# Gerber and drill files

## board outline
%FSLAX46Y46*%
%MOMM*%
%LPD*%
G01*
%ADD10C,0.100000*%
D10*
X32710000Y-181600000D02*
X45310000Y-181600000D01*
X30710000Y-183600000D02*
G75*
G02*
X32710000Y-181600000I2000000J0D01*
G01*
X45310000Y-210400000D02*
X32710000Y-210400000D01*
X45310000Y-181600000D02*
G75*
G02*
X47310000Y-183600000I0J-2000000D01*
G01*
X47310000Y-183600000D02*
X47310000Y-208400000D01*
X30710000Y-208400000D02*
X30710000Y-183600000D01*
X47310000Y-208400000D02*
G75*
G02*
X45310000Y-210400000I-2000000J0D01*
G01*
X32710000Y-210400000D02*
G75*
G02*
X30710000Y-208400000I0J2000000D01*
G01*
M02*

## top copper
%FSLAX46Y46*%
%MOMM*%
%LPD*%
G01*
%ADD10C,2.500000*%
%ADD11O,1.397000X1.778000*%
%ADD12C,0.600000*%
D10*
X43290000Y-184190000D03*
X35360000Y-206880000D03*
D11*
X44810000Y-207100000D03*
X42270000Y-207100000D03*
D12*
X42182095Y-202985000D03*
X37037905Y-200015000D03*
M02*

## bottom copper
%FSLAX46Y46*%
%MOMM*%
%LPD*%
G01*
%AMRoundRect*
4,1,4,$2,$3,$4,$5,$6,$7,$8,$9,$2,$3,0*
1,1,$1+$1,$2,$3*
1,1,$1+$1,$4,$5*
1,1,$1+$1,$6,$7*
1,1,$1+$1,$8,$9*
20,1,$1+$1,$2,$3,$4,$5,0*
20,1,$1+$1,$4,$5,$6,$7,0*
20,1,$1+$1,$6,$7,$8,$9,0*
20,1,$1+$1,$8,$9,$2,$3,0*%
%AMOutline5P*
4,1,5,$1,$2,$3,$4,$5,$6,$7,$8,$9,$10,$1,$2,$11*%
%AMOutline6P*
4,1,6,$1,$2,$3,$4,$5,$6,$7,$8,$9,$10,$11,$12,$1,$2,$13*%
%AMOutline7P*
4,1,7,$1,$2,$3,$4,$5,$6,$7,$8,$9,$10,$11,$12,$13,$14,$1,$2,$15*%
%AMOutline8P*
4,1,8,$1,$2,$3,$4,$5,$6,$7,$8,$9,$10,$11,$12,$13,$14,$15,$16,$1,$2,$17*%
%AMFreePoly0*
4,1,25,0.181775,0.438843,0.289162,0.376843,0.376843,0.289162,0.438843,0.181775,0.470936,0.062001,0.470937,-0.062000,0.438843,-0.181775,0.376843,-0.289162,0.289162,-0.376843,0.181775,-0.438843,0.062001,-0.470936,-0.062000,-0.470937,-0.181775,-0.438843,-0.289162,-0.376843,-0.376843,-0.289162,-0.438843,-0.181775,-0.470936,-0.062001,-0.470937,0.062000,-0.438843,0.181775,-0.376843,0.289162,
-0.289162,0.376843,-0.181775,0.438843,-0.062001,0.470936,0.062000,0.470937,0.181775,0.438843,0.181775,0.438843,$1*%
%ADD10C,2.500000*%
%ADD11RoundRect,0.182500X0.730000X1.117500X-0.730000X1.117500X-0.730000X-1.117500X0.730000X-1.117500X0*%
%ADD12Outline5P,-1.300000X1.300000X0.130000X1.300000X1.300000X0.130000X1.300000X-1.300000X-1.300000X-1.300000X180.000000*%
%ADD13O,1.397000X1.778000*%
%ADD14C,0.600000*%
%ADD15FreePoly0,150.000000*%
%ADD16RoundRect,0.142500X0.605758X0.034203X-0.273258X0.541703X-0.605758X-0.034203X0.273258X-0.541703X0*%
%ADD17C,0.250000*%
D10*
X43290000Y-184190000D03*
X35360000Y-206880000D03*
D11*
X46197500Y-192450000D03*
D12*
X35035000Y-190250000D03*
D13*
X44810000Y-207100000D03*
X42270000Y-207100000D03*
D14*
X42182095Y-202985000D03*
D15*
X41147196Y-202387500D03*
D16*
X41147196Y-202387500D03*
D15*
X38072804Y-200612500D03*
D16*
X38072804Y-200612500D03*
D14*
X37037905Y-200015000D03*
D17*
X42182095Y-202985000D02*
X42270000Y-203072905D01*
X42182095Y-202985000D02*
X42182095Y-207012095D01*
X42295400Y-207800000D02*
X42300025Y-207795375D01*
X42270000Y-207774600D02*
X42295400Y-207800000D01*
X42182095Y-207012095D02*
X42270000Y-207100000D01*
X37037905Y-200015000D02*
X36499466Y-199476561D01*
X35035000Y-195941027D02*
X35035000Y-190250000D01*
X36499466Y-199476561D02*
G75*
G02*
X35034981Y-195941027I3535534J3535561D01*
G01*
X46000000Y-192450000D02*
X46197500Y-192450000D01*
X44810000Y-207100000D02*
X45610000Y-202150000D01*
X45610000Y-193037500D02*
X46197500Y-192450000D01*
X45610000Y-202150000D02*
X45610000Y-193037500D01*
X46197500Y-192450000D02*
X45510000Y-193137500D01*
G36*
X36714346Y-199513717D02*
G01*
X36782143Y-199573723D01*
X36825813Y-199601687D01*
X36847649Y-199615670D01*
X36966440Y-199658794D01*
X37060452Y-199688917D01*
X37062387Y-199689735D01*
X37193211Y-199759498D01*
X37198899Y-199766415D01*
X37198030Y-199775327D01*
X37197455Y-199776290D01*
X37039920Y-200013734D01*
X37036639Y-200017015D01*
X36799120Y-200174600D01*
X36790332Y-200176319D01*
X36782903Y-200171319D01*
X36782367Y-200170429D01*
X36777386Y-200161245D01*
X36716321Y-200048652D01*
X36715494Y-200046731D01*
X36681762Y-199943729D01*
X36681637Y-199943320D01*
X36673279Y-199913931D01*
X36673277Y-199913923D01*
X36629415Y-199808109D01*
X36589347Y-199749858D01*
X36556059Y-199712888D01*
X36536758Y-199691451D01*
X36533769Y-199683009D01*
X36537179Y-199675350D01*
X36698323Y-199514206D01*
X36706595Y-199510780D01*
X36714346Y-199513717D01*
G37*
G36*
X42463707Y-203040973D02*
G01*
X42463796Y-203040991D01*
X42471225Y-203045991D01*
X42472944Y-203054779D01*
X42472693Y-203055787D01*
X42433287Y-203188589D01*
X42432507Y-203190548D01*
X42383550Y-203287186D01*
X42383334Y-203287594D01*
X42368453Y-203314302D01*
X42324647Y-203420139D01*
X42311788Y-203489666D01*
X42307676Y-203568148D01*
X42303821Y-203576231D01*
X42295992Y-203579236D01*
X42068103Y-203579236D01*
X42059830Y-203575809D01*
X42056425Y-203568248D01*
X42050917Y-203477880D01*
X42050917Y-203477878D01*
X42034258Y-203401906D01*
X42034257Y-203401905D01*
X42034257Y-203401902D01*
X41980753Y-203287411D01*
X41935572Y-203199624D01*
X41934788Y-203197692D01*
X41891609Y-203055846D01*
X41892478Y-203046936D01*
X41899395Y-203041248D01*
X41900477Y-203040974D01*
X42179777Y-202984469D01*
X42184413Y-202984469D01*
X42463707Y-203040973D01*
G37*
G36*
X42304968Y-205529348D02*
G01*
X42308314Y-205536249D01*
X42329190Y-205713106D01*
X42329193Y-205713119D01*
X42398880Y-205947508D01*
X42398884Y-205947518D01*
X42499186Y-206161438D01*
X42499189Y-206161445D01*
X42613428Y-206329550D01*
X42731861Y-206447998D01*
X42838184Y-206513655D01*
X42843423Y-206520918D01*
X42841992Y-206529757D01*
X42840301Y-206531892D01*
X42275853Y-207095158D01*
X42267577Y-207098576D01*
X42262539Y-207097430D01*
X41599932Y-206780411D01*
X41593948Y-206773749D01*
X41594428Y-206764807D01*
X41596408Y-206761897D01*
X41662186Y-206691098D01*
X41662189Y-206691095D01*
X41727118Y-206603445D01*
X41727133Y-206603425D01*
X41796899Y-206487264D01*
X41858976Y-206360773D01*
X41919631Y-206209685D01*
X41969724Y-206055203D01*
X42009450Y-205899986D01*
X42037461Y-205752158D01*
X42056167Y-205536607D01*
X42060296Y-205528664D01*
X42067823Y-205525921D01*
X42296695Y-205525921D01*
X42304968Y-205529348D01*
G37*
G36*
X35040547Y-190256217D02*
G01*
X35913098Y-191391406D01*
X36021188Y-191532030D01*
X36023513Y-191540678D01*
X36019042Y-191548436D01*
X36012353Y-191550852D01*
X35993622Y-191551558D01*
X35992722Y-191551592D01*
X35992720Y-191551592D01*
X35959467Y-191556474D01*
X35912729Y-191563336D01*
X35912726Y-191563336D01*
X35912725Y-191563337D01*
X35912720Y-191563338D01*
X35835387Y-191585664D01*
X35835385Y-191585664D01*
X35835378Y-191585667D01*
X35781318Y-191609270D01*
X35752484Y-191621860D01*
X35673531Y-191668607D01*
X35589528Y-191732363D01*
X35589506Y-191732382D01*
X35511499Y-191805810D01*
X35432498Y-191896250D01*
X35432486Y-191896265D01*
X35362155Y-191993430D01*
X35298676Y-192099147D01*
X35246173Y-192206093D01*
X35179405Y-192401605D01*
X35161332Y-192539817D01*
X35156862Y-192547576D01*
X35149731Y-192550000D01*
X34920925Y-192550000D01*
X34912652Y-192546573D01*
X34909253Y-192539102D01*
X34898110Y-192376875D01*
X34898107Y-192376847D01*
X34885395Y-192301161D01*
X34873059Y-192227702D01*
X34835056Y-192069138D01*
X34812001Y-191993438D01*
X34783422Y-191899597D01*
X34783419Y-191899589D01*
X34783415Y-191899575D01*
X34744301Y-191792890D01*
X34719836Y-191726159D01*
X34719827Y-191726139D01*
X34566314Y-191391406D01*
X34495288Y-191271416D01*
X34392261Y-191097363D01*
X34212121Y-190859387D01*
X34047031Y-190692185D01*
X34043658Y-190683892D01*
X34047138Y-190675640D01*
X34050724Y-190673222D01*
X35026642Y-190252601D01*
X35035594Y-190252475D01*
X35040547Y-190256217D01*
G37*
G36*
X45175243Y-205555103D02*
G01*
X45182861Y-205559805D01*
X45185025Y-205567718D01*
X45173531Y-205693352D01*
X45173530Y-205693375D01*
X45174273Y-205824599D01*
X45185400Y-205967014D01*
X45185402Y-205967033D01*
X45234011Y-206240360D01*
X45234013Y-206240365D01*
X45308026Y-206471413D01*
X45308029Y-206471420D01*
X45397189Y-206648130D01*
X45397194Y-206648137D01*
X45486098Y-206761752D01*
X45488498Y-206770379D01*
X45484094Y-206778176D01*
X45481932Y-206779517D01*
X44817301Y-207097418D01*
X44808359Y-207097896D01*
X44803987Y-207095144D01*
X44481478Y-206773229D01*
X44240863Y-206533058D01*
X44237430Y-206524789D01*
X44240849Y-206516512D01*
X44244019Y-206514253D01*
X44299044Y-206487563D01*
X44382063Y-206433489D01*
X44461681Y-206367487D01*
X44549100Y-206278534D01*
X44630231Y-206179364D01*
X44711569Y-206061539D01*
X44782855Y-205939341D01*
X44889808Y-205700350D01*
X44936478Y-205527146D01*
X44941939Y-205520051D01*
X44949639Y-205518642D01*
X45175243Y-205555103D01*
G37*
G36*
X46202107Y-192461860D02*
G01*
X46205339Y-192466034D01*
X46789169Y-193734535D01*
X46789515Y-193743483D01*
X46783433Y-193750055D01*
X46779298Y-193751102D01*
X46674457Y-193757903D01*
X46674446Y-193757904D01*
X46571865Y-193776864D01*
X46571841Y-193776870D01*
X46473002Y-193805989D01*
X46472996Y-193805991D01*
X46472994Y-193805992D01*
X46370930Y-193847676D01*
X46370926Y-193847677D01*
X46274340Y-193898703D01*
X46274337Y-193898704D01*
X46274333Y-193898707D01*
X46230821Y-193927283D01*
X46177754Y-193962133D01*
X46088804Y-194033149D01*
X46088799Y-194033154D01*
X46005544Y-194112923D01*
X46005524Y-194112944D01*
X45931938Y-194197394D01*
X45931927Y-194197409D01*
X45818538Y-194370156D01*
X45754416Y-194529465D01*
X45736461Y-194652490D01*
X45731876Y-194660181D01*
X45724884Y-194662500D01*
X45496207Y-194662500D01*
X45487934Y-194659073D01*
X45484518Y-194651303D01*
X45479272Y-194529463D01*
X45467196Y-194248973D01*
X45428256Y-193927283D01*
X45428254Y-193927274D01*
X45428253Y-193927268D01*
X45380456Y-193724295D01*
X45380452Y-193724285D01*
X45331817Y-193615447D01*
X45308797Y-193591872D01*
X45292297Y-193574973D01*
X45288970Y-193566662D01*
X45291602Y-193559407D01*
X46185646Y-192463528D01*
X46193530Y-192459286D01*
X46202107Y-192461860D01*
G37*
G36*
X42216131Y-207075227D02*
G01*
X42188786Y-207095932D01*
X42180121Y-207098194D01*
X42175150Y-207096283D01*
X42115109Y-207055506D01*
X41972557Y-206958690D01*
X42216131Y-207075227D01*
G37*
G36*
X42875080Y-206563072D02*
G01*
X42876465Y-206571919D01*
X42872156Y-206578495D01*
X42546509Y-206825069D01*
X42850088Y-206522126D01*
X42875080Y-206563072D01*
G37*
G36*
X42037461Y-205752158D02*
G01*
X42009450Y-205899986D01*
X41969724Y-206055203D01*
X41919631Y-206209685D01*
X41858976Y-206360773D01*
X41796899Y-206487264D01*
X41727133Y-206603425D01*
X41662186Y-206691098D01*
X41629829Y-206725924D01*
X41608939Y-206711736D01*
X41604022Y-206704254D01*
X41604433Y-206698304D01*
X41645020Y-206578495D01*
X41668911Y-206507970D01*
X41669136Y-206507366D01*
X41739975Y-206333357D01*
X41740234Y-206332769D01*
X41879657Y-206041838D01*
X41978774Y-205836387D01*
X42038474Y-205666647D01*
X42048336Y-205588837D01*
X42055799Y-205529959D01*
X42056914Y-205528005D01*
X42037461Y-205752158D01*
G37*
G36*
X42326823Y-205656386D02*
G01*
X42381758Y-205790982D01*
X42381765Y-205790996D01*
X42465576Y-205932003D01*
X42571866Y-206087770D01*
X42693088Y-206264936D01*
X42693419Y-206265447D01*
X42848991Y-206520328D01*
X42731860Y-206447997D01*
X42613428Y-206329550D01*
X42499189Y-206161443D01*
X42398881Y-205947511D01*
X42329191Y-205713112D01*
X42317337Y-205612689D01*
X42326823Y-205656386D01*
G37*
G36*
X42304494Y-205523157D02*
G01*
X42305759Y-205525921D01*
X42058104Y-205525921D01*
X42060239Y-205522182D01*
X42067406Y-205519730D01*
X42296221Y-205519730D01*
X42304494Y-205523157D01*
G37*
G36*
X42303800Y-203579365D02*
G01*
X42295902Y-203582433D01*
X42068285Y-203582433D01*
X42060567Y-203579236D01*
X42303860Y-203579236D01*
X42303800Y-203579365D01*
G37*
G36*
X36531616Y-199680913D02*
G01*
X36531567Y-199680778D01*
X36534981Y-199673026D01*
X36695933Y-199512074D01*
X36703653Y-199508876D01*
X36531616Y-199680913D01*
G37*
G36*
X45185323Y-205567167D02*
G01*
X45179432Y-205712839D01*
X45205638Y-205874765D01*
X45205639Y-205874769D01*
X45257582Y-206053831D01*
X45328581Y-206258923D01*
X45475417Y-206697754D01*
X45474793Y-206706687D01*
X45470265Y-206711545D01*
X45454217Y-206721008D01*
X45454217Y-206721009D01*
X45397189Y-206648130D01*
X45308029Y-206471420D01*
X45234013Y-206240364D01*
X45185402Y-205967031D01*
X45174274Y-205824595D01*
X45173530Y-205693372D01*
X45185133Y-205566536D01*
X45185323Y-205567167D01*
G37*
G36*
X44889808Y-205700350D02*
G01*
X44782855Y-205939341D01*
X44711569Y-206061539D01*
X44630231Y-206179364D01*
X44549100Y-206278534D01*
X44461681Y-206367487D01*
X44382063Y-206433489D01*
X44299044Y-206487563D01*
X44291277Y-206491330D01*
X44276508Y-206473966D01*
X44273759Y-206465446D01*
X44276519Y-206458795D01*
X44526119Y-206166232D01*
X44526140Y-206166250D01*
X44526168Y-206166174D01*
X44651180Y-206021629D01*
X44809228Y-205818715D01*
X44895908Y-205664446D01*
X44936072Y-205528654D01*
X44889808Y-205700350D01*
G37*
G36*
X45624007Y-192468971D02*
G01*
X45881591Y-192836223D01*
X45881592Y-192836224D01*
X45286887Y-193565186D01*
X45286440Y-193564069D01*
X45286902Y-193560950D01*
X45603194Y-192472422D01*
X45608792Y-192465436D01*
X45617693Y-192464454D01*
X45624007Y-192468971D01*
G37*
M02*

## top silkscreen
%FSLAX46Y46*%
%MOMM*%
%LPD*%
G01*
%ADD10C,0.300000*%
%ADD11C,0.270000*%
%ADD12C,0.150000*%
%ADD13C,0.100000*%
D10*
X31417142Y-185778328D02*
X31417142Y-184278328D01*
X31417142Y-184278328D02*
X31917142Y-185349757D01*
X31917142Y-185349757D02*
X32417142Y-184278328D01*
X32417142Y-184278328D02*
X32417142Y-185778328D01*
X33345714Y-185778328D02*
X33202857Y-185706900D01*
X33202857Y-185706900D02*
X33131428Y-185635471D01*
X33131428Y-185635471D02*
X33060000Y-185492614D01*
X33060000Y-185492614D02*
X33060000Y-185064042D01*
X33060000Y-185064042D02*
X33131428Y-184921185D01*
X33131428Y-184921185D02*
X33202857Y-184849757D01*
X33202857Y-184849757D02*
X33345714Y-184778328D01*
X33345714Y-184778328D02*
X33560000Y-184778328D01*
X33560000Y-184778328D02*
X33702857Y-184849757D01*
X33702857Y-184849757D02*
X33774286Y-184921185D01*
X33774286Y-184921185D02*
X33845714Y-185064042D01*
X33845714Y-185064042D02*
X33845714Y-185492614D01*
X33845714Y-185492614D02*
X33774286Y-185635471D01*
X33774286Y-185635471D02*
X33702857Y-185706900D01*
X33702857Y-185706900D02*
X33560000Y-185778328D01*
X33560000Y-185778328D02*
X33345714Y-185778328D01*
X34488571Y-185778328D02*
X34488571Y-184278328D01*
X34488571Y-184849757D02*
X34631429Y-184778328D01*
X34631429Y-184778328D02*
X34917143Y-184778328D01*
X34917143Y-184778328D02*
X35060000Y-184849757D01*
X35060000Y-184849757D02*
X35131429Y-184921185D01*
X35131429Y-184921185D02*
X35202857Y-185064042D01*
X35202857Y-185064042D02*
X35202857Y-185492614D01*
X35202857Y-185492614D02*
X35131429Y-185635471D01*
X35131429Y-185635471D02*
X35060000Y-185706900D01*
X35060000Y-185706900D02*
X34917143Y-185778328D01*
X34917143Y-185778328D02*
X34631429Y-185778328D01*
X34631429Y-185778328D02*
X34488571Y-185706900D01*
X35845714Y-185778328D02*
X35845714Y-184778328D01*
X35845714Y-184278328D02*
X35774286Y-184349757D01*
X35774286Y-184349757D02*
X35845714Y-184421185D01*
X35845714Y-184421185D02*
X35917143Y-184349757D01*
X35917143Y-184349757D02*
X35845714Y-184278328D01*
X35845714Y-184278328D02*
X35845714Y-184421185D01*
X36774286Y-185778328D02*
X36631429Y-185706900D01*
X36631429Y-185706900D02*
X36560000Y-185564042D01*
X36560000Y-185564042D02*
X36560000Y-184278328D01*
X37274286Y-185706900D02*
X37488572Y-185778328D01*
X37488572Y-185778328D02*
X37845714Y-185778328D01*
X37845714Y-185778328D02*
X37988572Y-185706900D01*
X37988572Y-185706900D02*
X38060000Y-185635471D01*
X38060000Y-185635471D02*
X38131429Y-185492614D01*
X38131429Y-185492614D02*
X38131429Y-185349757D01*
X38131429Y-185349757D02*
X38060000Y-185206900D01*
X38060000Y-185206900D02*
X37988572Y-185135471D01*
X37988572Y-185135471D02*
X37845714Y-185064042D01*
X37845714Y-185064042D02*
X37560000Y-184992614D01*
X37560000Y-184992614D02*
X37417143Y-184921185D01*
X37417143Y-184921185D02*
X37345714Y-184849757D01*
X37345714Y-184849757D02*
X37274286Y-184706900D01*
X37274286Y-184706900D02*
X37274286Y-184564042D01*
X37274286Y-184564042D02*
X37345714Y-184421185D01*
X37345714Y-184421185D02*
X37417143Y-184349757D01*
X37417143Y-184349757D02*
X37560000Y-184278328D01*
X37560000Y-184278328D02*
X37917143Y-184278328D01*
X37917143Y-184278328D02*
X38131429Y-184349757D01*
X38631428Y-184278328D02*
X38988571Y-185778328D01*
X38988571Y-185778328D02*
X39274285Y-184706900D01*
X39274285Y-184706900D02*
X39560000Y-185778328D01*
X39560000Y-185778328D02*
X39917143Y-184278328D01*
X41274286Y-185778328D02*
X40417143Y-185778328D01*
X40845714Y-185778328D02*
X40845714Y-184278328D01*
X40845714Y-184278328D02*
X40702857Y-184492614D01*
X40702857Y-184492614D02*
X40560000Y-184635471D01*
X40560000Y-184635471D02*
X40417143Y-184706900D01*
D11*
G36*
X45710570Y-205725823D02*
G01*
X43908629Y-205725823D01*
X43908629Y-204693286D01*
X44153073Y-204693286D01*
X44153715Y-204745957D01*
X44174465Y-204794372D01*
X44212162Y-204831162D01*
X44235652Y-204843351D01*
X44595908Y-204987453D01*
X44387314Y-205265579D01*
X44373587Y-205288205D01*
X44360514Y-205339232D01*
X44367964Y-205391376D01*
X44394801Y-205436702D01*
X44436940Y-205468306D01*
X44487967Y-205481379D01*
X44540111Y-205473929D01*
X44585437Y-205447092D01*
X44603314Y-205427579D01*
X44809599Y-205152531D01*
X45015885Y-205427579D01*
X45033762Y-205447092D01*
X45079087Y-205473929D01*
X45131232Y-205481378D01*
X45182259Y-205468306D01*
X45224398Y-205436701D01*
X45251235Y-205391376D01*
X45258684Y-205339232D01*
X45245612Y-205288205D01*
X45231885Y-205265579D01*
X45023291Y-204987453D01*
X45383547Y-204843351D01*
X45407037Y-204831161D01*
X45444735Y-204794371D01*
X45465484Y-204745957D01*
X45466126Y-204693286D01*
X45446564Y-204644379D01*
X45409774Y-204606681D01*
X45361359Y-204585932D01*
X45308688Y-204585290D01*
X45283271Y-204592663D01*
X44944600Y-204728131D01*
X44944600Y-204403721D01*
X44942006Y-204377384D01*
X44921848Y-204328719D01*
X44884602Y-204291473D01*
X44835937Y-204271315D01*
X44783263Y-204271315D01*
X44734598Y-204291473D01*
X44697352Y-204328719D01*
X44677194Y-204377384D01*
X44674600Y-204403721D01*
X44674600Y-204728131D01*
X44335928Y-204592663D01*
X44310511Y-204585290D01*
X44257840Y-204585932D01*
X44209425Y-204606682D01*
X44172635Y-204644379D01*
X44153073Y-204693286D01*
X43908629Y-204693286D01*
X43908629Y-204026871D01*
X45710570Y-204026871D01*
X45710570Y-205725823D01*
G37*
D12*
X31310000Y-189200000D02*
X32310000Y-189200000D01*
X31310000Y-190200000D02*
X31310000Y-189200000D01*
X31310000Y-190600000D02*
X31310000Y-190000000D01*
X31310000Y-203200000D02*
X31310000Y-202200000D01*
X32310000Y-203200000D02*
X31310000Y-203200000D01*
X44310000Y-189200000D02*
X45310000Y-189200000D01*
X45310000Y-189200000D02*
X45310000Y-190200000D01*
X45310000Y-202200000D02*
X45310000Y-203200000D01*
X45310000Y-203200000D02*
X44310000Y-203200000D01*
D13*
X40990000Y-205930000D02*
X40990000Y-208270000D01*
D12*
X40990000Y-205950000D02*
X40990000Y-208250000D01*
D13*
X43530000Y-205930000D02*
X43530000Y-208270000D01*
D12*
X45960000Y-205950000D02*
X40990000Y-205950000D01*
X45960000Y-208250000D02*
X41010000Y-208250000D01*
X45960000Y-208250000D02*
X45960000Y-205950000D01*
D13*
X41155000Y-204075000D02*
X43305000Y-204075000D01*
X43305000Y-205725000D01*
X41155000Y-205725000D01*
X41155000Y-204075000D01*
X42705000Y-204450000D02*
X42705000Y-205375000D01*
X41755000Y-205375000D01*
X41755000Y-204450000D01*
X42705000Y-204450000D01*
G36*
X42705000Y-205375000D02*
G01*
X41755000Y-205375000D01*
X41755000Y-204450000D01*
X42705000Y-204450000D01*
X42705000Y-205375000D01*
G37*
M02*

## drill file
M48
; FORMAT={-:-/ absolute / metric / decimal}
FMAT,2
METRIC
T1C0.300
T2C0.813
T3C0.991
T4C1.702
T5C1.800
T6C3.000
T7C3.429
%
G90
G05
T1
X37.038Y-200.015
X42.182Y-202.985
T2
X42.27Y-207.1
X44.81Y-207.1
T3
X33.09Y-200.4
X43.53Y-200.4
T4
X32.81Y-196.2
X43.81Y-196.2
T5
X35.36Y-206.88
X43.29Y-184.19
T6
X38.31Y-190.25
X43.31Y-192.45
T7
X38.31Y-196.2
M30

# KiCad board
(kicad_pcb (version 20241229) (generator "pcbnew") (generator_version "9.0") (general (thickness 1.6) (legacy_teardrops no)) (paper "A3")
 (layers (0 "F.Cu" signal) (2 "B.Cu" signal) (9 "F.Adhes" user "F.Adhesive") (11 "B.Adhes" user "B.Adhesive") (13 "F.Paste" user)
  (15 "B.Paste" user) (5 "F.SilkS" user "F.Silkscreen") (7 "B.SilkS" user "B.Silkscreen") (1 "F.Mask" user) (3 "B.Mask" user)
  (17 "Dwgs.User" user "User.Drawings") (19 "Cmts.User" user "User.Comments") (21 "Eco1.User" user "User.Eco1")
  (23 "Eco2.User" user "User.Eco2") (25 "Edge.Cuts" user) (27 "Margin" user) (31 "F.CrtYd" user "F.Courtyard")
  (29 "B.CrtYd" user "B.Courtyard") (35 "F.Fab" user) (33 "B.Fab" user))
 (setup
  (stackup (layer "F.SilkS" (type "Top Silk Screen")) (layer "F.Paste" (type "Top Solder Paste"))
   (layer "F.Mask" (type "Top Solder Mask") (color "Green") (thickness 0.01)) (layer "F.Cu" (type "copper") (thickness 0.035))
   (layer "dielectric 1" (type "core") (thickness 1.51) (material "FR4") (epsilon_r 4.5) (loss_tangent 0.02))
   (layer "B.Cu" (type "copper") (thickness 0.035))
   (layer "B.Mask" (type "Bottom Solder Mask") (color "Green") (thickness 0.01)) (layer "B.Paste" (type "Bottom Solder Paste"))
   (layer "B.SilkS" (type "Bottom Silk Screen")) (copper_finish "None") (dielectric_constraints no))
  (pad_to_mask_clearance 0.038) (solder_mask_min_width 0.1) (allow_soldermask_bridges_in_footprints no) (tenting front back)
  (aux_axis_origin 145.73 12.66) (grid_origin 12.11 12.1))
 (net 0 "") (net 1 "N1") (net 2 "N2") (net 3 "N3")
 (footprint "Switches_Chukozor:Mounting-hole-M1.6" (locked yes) (layer "F.Cu") (at 43.29 184.19)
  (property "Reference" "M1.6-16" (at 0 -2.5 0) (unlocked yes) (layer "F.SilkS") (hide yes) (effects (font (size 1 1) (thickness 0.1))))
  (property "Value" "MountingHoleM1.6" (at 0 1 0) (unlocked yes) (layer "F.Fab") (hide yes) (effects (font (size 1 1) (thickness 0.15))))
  (pad "" np_thru_hole circle (at 0 0) (size 2.5 2.5) (drill 1.8) (layers "*.Cu" "*.Mask") (clearance 0.2)))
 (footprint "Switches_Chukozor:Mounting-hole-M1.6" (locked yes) (layer "F.Cu") (at 35.36 206.88)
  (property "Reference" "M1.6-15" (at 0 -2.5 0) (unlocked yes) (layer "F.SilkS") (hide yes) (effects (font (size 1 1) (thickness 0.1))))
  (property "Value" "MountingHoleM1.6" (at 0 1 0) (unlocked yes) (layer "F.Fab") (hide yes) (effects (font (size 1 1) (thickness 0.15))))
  (pad "" np_thru_hole circle (at 0 0) (size 2.5 2.5) (drill 1.8) (layers "*.Cu" "*.Mask") (clearance 0.2)))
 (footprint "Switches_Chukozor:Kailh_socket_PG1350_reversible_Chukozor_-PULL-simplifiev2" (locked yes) (layer "F.Cu") (at 38.31 196.2 180)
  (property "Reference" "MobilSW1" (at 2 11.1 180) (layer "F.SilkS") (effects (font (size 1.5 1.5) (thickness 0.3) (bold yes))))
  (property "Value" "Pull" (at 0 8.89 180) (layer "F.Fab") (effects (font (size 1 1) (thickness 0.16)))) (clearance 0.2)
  (fp_line (start 7 7) (end 6 7) (stroke (width 0.15) (type solid)) (layer "F.SilkS"))
  (fp_line (start 7 6) (end 7 7) (stroke (width 0.15) (type solid)) (layer "F.SilkS"))
  (fp_line (start 7 5.6) (end 7 6.2) (stroke (width 0.15) (type solid)) (layer "F.SilkS"))
  (fp_line (start 7 -7) (end 7 -6) (stroke (width 0.15) (type solid)) (layer "F.SilkS"))
  (fp_line (start 6 -7) (end 7 -7) (stroke (width 0.15) (type solid)) (layer "F.SilkS"))
  (fp_line (start -6 7) (end -7 7) (stroke (width 0.15) (type solid)) (layer "F.SilkS"))
  (fp_line (start -7 7) (end -7 6) (stroke (width 0.15) (type solid)) (layer "F.SilkS"))
  (fp_line (start -7 -6) (end -7 -7) (stroke (width 0.15) (type solid)) (layer "F.SilkS"))
  (fp_line (start -7 -7) (end -6 -7) (stroke (width 0.15) (type solid)) (layer "F.SilkS"))
  (pad "" np_thru_hole circle (at -5.5 0 180) (size 1.7018 1.7018) (drill 1.7018) (layers "*.Cu" "*.Mask"))
  (pad "" np_thru_hole circle (at -5.22 -4.2 180) (size 0.9906 0.9906) (drill 0.9906) (layers "*.Cu" "*.Mask"))
  (pad "" np_thru_hole circle (at -5 3.75 180) (size 3 3) (drill 3) (layers "*.Cu" "*.Mask"))
  (pad "" np_thru_hole circle (at 0 0 180) (size 3.429 3.429) (drill 3.429) (layers "*.Cu" "*.Mask") (solder_mask_margin 0.1)
   (clearance 0.3))
  (pad "" np_thru_hole circle (at 0 5.95 180) (size 3 3) (drill 3) (layers "*.Cu" "*.Mask"))
  (pad "" np_thru_hole circle (at 5.22 -4.2 180) (size 0.9906 0.9906) (drill 0.9906) (layers "*.Cu" "*.Mask"))
  (pad "" np_thru_hole circle (at 5.5 0 180) (size 1.7018 1.7018) (drill 1.7018) (layers "*.Cu" "*.Mask"))
  (pad "1" smd roundrect (at -7.8875 3.75 180) (size 1.825 2.6) (layers "B.Cu" "B.Mask") (roundrect_rratio 0.1) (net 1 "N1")
   (teardrops (best_length_ratio 0.5) (max_length 1) (best_width_ratio 1) (max_width 2) (curved_edges yes) (filter_ratio 0.9) (enabled yes)
    (allow_two_segments yes) (prefer_zone_connections yes)))
  (pad "2" smd roundrect (at 3.275 5.95 180) (size 2.6 2.6) (layers "B.Cu" "B.Mask") (roundrect_rratio 0) (chamfer_ratio 0.45)
   (chamfer top_right) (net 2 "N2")
   (teardrops (best_length_ratio 0.5) (max_length 1) (best_width_ratio 1) (max_width 2) (curved_edges yes) (filter_ratio 0.9) (enabled yes)
    (allow_two_segments yes) (prefer_zone_connections yes))))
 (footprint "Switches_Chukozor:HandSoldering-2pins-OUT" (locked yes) (layer "F.Cu") (at 43.4146 207.1)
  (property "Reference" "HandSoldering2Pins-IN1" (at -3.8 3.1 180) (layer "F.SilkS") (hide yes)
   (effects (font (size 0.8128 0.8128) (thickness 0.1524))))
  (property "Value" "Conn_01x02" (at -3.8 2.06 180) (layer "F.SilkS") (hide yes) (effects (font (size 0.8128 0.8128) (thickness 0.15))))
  (fp_line (start -2.4246 -1.17) (end -2.4246 1.17) (stroke (width 0.1) (type default)) (layer "F.SilkS"))
  (fp_line (start -2.4246 -1.15) (end -2.4246 1.15) (stroke (width 0.15) (type solid)) (layer "F.SilkS"))
  (fp_line (start 0.1154 -1.17) (end 0.1154 1.17) (stroke (width 0.1) (type default)) (layer "F.SilkS"))
  (fp_line (start 2.5454 -1.15) (end -2.4246 -1.15) (stroke (width 0.15) (type solid)) (layer "F.SilkS"))
  (fp_line (start 2.5454 1.15) (end -2.4046 1.15) (stroke (width 0.15) (type solid)) (layer "F.SilkS"))
  (fp_line (start 2.5454 1.15) (end 2.5454 -1.15) (stroke (width 0.15) (type solid)) (layer "F.SilkS"))
  (fp_rect (start -0.1096 -3.025) (end -2.2596 -1.375) (stroke (width 0.1) (type default)) (fill no) (layer "F.SilkS"))
  (fp_poly
   (pts (xy -0.7096 -2.65) (xy -0.7096 -1.725) (xy -1.6596 -1.725) (xy -1.6596 -2.65)) (stroke (width 0.1) (type solid)) (fill yes)
   (layer "F.SilkS"))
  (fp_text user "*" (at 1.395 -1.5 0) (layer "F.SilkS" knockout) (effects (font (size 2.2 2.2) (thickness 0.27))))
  (pad "1" thru_hole oval (at 1.3954 0) (size 1.397 1.778) (drill 0.8128) (layers "*.Cu" "*.Mask") (remove_unused_layers no) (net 1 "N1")
   (teardrops (best_length_ratio 0.5) (max_length 1) (best_width_ratio 1) (max_width 2) (curved_edges yes) (filter_ratio 0.9) (enabled yes)
    (allow_two_segments yes) (prefer_zone_connections yes)))
  (pad "2" thru_hole oval (at -1.1446 0) (size 1.397 1.778) (drill 0.8128) (layers "*.Cu" "*.Mask") (remove_unused_layers no) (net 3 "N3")
   (teardrops (best_length_ratio 0.5) (max_length 1) (best_width_ratio 1) (max_width 2) (curved_edges yes) (filter_ratio 0.9) (enabled yes)
    (allow_two_segments yes) (prefer_zone_connections yes))))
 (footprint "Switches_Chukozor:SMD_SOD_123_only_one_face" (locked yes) (layer "F.Cu") (at 39.61 201.5 150)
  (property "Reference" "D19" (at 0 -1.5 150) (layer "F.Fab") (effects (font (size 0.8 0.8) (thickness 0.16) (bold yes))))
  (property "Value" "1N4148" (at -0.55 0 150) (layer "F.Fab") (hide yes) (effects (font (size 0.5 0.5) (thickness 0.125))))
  (pad "1" thru_hole circle (at -2.97 0 150) (size 0.6 0.6) (drill 0.3) (layers "*.Cu") (remove_unused_layers no) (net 3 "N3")
   (teardrops (best_length_ratio 0.5) (max_length 1) (best_width_ratio 1) (max_width 2) (curved_edges yes) (filter_ratio 0.9) (enabled yes)
    (allow_two_segments yes) (prefer_zone_connections yes)))
  (pad "1" smd custom (at -1.775001 0 150) (size 0.95 0.95) (layers "B.Cu") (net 3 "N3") (thermal_bridge_angle 90)
   (options (clearance outline) (anchor circle)) (primitives)
   (teardrops (best_length_ratio 0.5) (max_length 1) (best_width_ratio 1) (max_width 2) (curved_edges no) (filter_ratio 0.9) (enabled no)
    (allow_two_segments no) (prefer_zone_connections yes)))
  (pad "1" smd roundrect (at -1.775001 0 150) (size 1.3 0.95) (layers "B.Cu" "B.Mask") (roundrect_rratio 0.15) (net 3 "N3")
   (teardrops (best_length_ratio 0.5) (max_length 1) (best_width_ratio 1) (max_width 2) (curved_edges yes) (filter_ratio 0.9) (enabled yes)
    (allow_two_segments yes) (prefer_zone_connections yes)))
  (pad "2" smd custom (at 1.775001 0 150) (size 0.95 0.95) (layers "B.Cu") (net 2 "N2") (thermal_bridge_angle 90)
   (options (clearance outline) (anchor circle)) (primitives)
   (teardrops (best_length_ratio 0.5) (max_length 1) (best_width_ratio 1) (max_width 2) (curved_edges no) (filter_ratio 0.9) (enabled no)
    (allow_two_segments no) (prefer_zone_connections yes)))
  (pad "2" smd roundrect (at 1.775001 0 150) (size 1.3 0.95) (layers "B.Cu" "B.Mask") (roundrect_rratio 0.15) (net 2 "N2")
   (teardrops (best_length_ratio 0.5) (max_length 1) (best_width_ratio 1) (max_width 2) (curved_edges yes) (filter_ratio 0.9) (enabled yes)
    (allow_two_segments yes) (prefer_zone_connections yes)))
  (pad "2" thru_hole circle (at 2.97 0 150) (size 0.6 0.6) (drill 0.3) (layers "*.Cu") (remove_unused_layers no) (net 2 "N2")
   (teardrops (best_length_ratio 0.5) (max_length 1) (best_width_ratio 1) (max_width 2) (curved_edges yes) (filter_ratio 0.9) (enabled yes)
    (allow_two_segments yes) (prefer_zone_connections yes))))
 (gr_line (start 32.71 181.6) (end 45.31 181.6) (stroke (width 0.1) (type default)) (locked yes) (layer "Edge.Cuts"))
 (gr_arc (start 30.71 183.6) (mid 31.295786 182.185786) (end 32.71 181.6) (stroke (width 0.1) (type default)) (locked yes)
  (layer "Edge.Cuts"))
 (gr_line (start 45.31 210.4) (end 32.71 210.4) (stroke (width 0.1) (type default)) (locked yes) (layer "Edge.Cuts"))
 (gr_arc (start 45.31 181.6) (mid 46.724214 182.185786) (end 47.31 183.6) (stroke (width 0.1) (type default)) (locked yes)
  (layer "Edge.Cuts"))
 (gr_line (start 47.31 183.6) (end 47.31 208.4) (stroke (width 0.1) (type default)) (locked yes) (layer "Edge.Cuts"))
 (gr_line (start 30.71 208.4) (end 30.71 183.6) (stroke (width 0.1) (type default)) (locked yes) (layer "Edge.Cuts"))
 (gr_arc (start 47.31 208.4) (mid 46.724214 209.814214) (end 45.31 210.4) (stroke (width 0.1) (type default)) (locked yes)
  (layer "Edge.Cuts"))
 (gr_arc (start 32.71 210.4) (mid 31.295786 209.814214) (end 30.71 208.4) (stroke (width 0.1) (type default)) (locked yes)
  (layer "Edge.Cuts"))
 (segment (start 42.182095 202.985) (end 42.27 203.072905) (width 0.25) (layer "B.Cu") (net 3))
 (segment (start 42.182095 202.985) (end 42.182095 207.012095) (width 0.25) (layer "B.Cu") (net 3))
 (segment (start 42.2954 207.8) (end 42.300025 207.795375) (width 0.25) (layer "B.Cu") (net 3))
 (segment (start 42.27 207.7746) (end 42.2954 207.8) (width 0.25) (layer "B.Cu") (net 3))
 (segment (start 42.182095 207.012095) (end 42.27 207.1) (width 0.25) (layer "B.Cu") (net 3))
 (segment (start 37.037905 200.015) (end 36.499466 199.476561) (width 0.25) (layer "B.Cu") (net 2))
 (segment (start 35.035 195.941027) (end 35.035 190.25) (width 0.25) (layer "B.Cu") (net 2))
 (arc (start 36.499466 199.476561) (mid 35.415602 197.854444) (end 35.035 195.941027) (width 0.25) (layer "B.Cu") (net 2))
 (segment (start 46 192.45) (end 46.1975 192.45) (width 0.25) (layer "B.Cu") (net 1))
 (segment (start 44.81 207.1) (end 45.61 202.15) (width 0.25) (layer "B.Cu") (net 1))
 (segment (start 45.61 193.0375) (end 46.1975 192.45) (width 0.25) (layer "B.Cu") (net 1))
 (segment (start 45.61 202.15) (end 45.61 193.0375) (width 0.25) (layer "B.Cu") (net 1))
 (segment (start 46.1975 192.45) (end 45.51 193.1375) (width 0.25) (layer "B.Cu") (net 1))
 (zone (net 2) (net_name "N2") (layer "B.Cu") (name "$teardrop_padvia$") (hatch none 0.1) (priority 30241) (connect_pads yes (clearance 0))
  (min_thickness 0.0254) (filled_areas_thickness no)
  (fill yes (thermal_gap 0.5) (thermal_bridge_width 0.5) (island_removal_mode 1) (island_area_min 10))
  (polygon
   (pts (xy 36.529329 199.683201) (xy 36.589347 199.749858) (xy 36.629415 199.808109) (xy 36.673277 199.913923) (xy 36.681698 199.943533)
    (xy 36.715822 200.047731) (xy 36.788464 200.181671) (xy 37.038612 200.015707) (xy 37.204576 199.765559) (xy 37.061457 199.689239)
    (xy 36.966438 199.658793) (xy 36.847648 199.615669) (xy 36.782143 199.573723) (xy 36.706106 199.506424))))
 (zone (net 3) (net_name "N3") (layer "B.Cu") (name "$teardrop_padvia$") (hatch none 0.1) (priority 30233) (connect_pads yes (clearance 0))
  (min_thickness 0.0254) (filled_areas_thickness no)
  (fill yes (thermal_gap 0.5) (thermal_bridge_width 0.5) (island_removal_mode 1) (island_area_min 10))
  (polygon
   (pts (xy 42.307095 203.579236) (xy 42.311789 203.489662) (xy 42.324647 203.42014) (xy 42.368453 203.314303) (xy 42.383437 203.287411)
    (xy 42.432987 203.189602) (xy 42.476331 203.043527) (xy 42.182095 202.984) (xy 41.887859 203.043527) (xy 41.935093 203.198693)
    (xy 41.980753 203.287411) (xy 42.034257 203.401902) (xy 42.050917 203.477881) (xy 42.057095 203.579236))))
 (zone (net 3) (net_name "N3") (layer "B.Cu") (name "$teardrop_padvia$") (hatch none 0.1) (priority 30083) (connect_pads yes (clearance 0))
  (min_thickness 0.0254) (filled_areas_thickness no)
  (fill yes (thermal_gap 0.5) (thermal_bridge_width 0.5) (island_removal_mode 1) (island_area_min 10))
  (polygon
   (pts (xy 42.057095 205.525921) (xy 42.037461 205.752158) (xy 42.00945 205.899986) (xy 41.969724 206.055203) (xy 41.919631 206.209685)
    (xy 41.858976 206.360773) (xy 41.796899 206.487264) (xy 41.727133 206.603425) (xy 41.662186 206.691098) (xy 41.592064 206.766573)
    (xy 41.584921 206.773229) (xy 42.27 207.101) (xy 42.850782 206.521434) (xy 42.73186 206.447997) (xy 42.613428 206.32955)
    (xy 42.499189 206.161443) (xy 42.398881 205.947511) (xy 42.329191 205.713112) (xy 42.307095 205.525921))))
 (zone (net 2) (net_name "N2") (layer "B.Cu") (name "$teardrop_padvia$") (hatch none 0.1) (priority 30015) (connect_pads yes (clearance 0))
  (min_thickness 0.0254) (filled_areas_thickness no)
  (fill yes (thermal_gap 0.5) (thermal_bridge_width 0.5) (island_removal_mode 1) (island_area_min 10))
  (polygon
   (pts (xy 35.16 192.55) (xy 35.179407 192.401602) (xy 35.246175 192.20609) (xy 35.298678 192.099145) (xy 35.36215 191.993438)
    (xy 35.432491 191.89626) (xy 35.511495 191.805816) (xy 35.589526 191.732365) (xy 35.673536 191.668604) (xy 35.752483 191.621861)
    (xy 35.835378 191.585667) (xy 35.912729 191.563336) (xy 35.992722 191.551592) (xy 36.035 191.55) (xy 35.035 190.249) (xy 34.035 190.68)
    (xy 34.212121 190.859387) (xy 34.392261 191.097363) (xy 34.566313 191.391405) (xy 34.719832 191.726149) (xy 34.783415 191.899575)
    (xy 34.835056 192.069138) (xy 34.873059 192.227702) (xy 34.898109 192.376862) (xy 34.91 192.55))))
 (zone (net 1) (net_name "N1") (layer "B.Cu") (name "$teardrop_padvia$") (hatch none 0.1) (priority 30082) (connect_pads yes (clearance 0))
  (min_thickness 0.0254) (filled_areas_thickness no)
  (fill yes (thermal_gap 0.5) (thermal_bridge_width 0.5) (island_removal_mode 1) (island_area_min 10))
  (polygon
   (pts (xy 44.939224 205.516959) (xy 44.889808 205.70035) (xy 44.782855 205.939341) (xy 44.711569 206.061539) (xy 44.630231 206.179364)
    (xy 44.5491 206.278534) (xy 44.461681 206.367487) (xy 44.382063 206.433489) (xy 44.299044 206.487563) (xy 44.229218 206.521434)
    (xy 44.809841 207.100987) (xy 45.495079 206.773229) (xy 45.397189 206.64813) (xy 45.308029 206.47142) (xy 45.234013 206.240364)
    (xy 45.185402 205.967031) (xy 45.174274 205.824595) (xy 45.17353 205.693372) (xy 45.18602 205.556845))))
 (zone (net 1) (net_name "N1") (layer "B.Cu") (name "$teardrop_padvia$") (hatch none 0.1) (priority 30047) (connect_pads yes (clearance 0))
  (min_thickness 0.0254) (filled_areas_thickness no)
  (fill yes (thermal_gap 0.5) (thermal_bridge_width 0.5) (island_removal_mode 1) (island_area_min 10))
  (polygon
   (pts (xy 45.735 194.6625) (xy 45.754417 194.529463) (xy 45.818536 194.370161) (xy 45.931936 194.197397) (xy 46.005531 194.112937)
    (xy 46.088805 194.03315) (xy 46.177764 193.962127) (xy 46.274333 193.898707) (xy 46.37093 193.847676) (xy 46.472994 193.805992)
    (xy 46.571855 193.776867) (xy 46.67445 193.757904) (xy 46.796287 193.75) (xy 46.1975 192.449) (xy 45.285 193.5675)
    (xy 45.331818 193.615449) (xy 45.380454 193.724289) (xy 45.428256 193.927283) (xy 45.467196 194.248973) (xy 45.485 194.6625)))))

